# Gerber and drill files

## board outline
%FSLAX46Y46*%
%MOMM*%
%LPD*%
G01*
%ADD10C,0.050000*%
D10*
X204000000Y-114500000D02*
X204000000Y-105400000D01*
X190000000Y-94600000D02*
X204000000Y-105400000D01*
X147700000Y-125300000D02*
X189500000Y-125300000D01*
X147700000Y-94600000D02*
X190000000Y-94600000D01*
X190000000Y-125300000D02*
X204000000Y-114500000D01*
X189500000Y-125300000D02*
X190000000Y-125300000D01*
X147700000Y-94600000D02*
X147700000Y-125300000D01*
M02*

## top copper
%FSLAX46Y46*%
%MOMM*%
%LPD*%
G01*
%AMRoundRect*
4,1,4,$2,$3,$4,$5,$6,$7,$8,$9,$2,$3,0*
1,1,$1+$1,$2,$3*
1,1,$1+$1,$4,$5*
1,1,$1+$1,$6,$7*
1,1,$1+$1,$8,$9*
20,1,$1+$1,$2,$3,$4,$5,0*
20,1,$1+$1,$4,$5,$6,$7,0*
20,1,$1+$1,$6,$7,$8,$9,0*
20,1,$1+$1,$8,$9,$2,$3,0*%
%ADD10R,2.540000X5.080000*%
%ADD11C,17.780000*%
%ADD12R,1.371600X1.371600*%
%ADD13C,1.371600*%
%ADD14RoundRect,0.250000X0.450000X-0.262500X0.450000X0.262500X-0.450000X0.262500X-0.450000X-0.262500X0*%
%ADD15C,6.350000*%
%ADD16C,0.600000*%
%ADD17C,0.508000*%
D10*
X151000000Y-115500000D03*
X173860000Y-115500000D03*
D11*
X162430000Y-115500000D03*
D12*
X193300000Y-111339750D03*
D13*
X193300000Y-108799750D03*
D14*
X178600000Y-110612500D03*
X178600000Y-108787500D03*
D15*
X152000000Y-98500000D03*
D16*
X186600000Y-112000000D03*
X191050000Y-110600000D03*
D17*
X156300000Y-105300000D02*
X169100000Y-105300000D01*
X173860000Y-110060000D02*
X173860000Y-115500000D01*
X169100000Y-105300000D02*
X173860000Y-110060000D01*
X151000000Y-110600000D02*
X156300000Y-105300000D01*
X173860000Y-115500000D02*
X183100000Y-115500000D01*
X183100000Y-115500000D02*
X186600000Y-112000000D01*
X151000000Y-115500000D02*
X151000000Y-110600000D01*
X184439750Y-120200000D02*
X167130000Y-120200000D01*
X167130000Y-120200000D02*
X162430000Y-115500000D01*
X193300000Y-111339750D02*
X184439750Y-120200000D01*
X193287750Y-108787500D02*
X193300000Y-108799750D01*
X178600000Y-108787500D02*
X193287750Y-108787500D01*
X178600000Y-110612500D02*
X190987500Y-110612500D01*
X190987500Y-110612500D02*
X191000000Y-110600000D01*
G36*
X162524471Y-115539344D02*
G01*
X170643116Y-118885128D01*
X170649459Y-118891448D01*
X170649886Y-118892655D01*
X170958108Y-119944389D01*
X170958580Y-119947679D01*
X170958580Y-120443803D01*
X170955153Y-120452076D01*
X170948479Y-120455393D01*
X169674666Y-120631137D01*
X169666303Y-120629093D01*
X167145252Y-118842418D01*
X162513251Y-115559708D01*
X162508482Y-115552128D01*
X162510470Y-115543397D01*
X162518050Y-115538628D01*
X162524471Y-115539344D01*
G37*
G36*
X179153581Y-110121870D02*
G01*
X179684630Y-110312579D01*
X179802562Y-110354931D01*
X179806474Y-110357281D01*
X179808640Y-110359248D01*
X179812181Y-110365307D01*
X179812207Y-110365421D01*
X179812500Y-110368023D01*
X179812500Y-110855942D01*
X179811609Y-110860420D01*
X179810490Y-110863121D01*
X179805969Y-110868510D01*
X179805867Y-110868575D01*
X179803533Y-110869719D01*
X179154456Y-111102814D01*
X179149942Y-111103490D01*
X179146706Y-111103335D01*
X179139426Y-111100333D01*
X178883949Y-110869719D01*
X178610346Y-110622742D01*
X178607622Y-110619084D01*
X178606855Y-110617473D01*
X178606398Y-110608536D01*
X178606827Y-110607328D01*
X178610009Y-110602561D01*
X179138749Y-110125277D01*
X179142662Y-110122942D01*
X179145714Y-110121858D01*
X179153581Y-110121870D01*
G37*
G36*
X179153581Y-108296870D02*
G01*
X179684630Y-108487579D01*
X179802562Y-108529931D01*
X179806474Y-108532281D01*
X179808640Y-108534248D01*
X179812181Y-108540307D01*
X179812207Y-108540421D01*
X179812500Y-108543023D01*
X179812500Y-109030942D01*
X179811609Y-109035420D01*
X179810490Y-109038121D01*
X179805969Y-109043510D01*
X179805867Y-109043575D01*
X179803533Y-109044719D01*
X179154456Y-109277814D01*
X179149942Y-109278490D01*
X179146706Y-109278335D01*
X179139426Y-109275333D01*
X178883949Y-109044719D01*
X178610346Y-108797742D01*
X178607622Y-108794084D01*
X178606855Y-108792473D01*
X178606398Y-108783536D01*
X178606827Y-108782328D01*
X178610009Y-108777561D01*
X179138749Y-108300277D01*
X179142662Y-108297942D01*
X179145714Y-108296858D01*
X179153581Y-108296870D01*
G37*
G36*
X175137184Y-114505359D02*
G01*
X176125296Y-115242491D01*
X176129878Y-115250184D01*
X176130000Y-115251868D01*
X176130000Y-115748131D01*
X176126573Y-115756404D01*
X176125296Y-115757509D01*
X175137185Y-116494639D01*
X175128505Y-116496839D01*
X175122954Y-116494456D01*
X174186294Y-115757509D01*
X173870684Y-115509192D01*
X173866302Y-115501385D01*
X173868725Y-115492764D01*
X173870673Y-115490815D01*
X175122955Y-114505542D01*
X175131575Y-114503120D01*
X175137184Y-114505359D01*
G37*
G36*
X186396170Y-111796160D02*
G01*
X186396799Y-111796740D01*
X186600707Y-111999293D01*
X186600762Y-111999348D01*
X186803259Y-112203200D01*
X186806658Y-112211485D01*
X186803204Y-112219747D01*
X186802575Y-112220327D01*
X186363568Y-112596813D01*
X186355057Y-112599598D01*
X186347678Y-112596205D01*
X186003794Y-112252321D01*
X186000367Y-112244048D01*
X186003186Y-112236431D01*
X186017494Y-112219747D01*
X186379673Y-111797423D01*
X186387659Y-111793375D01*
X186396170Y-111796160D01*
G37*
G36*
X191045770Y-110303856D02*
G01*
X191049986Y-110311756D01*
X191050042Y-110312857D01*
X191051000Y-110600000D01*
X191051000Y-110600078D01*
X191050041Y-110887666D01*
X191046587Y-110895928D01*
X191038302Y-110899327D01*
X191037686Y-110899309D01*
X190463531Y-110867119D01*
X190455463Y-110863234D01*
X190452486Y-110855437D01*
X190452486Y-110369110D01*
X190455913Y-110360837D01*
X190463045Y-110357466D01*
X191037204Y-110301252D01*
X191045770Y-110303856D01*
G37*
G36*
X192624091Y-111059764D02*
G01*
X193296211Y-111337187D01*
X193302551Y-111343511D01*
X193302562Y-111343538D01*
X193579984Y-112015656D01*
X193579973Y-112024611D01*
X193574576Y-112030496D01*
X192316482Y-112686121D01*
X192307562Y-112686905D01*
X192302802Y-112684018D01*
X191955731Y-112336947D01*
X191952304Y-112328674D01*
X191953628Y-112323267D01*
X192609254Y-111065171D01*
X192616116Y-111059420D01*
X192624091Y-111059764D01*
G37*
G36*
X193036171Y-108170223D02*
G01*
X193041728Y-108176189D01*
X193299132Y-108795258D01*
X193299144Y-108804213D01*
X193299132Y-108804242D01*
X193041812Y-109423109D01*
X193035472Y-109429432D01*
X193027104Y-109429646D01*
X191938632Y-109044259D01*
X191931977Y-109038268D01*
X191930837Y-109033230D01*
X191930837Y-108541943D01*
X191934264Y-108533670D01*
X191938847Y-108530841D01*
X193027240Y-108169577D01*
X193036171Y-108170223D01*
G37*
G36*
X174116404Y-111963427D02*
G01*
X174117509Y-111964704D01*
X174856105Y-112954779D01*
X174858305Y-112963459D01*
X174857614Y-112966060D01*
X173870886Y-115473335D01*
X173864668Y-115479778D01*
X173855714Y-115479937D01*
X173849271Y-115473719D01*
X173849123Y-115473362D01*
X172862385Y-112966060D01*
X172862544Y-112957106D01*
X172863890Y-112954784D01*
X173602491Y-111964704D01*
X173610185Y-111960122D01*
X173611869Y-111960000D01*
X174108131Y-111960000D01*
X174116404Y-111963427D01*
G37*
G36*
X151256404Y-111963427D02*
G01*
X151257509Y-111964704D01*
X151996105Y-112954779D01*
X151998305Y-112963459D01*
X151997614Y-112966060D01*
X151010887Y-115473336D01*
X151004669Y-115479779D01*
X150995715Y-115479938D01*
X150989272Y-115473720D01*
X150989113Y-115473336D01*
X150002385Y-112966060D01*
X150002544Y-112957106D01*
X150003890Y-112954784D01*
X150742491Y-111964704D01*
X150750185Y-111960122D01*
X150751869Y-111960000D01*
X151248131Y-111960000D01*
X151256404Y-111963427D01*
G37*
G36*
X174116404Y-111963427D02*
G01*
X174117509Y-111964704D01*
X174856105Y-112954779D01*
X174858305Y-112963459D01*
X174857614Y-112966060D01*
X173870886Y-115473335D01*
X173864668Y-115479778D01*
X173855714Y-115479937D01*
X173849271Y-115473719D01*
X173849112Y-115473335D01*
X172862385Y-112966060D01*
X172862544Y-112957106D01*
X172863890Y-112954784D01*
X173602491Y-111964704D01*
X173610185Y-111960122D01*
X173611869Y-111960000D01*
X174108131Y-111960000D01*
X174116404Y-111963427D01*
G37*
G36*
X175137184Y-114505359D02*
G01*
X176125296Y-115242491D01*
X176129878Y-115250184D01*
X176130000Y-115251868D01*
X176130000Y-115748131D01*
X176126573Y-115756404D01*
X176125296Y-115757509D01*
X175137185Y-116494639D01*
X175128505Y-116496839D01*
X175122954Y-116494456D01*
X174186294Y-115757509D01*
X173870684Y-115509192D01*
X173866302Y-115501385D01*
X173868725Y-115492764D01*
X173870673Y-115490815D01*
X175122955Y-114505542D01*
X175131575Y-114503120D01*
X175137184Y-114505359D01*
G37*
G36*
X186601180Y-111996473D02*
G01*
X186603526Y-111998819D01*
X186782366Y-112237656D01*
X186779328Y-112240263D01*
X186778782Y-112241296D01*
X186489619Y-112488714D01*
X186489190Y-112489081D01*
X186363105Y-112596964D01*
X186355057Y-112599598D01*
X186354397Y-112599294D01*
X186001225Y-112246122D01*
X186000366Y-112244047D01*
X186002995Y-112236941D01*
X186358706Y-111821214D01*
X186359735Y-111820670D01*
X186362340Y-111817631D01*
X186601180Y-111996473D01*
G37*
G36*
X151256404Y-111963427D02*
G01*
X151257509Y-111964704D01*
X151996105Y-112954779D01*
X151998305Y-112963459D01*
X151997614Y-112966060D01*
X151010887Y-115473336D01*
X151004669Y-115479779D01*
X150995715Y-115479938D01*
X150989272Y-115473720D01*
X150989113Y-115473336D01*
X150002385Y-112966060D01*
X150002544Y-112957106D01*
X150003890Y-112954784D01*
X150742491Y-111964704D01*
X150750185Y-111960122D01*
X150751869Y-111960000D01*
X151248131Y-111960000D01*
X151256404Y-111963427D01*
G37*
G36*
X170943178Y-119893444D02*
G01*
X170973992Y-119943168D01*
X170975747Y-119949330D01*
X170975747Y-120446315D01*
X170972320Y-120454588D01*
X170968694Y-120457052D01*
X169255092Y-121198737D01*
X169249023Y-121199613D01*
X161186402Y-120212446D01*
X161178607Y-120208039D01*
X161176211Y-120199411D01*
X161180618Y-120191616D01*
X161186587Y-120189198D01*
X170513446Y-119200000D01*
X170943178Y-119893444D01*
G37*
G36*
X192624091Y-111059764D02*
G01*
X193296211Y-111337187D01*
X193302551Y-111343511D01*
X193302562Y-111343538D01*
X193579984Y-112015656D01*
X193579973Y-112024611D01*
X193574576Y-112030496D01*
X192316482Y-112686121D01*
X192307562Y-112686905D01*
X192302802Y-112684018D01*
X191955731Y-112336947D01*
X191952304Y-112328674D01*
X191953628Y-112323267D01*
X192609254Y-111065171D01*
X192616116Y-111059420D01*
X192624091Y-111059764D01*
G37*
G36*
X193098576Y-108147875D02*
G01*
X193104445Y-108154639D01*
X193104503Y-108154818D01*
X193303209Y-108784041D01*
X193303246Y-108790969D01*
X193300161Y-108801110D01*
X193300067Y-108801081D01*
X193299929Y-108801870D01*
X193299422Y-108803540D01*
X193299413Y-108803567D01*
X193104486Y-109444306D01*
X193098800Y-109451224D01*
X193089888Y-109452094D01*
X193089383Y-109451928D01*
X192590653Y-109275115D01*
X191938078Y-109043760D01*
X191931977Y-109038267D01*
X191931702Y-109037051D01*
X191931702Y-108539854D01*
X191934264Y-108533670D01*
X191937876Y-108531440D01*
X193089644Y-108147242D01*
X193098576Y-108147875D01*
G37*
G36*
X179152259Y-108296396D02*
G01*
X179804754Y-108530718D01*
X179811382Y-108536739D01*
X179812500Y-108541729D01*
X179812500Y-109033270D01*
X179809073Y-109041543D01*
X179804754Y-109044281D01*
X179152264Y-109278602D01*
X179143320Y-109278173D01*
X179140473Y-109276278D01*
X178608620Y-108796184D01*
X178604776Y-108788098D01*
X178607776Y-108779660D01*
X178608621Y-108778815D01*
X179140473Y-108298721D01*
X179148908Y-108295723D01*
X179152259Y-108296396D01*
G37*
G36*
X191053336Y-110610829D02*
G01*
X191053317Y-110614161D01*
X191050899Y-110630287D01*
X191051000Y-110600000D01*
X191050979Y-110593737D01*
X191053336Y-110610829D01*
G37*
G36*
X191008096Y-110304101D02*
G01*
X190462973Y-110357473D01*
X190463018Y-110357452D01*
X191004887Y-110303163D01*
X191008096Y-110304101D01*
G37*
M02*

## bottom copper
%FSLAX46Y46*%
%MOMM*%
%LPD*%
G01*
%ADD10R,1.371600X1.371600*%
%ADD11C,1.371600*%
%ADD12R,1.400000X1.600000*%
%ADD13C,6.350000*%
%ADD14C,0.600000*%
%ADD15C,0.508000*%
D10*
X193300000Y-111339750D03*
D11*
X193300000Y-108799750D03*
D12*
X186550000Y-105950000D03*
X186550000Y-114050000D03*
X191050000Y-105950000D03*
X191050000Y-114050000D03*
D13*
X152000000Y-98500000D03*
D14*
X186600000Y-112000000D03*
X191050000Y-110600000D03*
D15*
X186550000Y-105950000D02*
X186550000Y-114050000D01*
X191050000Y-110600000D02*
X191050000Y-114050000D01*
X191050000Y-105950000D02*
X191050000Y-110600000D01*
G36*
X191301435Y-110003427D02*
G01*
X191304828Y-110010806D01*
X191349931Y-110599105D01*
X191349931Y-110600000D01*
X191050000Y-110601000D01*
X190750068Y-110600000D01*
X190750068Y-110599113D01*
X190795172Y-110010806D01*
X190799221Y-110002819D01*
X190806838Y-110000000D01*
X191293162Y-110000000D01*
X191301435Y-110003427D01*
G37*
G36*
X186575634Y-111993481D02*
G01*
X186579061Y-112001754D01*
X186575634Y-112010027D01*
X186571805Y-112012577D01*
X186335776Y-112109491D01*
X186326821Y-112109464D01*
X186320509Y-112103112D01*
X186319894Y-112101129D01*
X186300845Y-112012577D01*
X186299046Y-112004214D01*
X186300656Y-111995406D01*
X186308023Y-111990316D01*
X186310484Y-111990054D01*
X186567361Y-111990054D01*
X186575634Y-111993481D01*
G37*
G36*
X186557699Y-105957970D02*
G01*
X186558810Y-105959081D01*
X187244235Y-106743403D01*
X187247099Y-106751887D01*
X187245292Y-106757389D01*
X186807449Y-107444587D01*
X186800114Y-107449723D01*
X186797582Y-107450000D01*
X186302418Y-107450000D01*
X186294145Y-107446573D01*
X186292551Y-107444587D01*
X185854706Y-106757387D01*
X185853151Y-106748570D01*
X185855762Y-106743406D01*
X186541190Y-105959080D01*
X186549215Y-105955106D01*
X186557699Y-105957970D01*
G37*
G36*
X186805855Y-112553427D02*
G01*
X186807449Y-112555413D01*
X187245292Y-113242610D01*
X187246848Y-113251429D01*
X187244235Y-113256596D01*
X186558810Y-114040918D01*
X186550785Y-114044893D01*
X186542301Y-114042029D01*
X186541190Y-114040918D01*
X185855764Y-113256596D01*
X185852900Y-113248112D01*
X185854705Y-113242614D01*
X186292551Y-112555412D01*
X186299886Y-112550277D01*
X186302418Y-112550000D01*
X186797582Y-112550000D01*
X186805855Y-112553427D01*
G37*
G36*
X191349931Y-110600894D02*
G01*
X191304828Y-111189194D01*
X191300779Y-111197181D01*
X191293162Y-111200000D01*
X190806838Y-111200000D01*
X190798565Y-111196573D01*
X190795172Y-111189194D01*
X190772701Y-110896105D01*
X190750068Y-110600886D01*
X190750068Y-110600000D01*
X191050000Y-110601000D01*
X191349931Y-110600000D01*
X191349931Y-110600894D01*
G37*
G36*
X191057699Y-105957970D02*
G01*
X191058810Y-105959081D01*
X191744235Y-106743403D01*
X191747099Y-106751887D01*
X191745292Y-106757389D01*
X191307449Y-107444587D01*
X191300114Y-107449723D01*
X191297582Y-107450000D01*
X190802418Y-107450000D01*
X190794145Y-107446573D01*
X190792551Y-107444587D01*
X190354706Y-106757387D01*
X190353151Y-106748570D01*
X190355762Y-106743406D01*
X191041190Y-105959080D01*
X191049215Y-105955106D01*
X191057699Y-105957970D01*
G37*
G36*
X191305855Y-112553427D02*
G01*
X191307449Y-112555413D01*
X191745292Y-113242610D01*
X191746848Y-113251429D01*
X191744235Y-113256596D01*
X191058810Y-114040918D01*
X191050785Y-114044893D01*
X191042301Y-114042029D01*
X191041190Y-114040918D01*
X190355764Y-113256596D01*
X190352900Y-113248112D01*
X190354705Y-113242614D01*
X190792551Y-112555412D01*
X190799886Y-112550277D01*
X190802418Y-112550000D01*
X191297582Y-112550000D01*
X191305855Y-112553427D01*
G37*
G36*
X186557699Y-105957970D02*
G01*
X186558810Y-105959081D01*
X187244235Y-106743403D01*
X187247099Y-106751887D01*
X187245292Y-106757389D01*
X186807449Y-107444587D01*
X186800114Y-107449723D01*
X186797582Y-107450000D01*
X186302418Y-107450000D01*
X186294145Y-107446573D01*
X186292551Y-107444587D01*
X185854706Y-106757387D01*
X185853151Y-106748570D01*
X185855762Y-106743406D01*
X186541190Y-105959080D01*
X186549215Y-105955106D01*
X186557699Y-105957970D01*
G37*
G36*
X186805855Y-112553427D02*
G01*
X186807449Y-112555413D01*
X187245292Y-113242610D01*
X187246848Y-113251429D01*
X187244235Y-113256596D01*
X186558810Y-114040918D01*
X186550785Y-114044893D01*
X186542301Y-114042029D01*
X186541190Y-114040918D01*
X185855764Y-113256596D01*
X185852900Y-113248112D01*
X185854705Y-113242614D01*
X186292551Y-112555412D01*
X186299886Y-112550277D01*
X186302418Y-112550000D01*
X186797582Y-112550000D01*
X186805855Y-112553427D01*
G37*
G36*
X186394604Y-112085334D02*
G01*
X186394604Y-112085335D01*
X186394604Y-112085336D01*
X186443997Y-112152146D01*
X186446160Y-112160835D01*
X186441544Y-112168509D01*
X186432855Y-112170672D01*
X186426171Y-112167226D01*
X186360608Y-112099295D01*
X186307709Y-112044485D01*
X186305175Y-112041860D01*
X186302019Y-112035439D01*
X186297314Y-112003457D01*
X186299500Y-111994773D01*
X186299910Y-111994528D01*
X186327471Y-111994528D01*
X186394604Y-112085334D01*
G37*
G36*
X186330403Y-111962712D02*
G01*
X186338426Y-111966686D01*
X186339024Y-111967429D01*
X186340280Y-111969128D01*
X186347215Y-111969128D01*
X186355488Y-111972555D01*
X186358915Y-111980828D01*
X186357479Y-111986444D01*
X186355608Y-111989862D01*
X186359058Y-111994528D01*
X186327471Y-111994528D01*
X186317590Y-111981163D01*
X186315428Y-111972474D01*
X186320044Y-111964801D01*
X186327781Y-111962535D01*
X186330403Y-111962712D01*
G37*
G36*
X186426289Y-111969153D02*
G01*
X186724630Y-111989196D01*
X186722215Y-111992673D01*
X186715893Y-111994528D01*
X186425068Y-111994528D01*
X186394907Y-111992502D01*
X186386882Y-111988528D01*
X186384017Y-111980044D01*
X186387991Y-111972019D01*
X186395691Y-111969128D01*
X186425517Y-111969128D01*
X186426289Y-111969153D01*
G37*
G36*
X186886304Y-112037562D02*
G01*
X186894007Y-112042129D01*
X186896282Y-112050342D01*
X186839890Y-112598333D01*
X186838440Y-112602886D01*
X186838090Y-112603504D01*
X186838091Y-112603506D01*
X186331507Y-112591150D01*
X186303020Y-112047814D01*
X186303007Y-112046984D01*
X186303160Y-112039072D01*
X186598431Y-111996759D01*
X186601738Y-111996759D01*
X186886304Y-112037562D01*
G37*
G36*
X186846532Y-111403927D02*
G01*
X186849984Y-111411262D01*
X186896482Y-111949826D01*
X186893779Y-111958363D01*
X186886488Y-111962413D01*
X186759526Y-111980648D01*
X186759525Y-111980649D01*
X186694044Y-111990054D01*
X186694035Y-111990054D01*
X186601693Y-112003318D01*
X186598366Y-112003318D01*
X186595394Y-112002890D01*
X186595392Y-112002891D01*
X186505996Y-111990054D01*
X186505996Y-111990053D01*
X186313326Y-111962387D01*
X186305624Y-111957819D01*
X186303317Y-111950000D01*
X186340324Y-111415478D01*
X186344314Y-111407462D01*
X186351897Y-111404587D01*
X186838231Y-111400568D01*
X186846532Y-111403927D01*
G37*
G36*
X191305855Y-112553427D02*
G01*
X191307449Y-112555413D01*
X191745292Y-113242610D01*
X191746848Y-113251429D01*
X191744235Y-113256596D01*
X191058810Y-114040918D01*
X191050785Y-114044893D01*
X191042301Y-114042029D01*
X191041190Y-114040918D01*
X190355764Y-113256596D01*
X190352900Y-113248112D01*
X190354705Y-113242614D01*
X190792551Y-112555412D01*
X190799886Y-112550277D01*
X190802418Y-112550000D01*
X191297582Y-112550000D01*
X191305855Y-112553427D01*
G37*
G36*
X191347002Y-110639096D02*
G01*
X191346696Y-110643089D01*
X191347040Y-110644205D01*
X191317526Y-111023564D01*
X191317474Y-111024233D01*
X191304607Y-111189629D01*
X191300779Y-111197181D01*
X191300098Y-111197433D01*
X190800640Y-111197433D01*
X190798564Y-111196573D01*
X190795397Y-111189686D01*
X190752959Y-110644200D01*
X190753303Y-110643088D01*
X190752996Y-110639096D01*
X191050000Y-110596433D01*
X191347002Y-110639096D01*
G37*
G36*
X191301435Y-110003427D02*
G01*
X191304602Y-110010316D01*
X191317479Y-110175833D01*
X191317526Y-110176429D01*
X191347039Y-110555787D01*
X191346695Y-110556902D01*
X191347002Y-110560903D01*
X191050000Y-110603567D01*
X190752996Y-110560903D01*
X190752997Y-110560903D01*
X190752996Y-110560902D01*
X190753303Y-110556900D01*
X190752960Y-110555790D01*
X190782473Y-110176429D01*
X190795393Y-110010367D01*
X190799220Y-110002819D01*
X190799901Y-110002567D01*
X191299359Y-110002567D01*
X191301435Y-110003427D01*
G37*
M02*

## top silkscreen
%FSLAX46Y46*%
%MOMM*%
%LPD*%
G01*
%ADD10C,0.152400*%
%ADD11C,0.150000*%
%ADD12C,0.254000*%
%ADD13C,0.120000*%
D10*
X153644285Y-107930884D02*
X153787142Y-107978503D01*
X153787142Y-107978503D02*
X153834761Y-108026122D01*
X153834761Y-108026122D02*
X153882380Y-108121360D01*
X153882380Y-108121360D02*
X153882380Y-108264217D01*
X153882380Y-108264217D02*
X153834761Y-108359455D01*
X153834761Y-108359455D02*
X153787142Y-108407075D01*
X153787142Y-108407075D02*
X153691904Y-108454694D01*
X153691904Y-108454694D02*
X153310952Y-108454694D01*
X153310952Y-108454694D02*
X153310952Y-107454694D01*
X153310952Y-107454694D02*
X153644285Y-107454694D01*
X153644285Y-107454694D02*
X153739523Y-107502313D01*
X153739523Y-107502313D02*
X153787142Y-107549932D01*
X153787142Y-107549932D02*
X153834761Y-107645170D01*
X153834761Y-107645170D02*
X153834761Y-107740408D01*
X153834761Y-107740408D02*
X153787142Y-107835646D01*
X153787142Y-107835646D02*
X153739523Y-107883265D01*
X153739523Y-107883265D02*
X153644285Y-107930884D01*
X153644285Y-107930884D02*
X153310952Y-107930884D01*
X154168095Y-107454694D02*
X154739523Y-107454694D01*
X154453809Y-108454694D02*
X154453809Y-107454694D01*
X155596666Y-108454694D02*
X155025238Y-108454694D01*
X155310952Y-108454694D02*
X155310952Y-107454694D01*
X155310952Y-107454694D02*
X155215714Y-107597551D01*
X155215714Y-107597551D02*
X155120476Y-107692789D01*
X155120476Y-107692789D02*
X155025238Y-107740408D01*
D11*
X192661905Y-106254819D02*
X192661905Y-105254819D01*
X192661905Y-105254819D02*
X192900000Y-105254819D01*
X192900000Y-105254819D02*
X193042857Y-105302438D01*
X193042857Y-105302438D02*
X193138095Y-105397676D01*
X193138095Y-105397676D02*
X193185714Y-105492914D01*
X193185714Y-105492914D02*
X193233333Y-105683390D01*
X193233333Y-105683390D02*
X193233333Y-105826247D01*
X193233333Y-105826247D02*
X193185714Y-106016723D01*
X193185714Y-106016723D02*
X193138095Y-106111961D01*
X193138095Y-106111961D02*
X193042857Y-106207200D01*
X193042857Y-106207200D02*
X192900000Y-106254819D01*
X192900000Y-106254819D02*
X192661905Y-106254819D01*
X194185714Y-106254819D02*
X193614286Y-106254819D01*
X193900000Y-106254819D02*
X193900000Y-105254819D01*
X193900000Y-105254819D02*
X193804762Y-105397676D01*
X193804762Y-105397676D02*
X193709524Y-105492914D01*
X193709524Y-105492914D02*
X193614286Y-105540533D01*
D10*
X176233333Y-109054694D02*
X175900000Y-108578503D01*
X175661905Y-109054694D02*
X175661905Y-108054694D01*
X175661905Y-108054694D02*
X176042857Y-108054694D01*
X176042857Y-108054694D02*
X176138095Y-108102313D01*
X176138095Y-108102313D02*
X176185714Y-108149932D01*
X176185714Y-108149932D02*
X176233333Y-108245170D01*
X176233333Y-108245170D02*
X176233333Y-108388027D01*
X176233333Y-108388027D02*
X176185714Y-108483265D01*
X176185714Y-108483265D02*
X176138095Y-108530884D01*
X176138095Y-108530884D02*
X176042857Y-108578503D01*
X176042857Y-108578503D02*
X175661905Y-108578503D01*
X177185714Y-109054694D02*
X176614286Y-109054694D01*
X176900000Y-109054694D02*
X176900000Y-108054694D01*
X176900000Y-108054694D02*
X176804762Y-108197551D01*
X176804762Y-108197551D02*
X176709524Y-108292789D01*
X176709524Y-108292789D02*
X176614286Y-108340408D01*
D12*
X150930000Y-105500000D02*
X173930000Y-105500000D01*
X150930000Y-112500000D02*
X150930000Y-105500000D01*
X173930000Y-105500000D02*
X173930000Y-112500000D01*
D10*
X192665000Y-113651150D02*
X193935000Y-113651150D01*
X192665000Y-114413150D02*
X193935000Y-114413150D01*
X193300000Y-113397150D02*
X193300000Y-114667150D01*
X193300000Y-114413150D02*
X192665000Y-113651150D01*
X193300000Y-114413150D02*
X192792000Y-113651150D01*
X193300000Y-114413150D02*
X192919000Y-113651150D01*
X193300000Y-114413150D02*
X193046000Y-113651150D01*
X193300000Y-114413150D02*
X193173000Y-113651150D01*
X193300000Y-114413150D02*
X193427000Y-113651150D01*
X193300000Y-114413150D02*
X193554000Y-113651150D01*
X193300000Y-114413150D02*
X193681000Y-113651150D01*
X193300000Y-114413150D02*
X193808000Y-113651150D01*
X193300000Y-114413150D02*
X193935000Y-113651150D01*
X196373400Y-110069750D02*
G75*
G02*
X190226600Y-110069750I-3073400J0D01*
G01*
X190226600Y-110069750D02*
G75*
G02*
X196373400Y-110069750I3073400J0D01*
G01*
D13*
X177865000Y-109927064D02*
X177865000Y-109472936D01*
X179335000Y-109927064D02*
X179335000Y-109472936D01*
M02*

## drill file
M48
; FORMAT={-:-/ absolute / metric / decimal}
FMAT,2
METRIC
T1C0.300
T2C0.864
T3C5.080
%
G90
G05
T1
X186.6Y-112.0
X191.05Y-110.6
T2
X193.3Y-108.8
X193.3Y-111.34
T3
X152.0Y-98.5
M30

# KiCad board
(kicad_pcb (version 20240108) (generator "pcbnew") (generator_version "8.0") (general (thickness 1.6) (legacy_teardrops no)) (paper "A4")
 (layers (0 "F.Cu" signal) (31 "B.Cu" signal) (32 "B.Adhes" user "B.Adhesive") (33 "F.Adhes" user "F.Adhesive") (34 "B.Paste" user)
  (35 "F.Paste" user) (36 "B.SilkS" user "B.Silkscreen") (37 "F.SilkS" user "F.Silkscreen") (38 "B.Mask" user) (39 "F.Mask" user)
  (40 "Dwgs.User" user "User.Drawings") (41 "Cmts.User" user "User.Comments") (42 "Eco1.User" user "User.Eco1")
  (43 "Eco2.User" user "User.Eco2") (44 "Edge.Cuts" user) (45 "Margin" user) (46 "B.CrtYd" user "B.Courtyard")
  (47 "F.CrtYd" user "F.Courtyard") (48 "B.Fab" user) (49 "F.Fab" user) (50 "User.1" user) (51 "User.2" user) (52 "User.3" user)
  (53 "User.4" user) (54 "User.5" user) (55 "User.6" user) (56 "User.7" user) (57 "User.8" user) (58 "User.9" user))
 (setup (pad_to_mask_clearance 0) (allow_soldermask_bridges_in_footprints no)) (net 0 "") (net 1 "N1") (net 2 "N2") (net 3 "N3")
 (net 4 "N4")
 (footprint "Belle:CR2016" (layer "F.Cu") (at 162.43 115.5)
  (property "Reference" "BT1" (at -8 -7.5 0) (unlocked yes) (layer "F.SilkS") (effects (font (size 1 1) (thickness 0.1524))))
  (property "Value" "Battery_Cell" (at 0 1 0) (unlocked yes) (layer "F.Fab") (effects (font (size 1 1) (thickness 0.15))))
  (fp_line (start -11.5 -10) (end 11.5 -10) (stroke (width 0.254) (type default)) (layer "F.SilkS"))
  (fp_line (start -11.5 -3) (end -11.5 -10) (stroke (width 0.254) (type default)) (layer "F.SilkS"))
  (fp_line (start 11.5 -10) (end 11.5 -3) (stroke (width 0.254) (type default)) (layer "F.SilkS"))
  (pad "1" smd rect (at -11.43 0) (size 2.54 5.08) (layers "F.Cu" "F.Paste" "F.Mask") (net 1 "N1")
   (teardrops (best_length_ratio 0.5) (max_length 1) (best_width_ratio 1) (max_width 2) (curve_points 0) (filter_ratio 0.9) (enabled yes)
    (allow_two_segments yes) (prefer_zone_connections yes)))
  (pad "1" smd rect (at 11.43 0) (size 2.54 5.08) (layers "F.Cu" "F.Paste" "F.Mask") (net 1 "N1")
   (teardrops (best_length_ratio 0.5) (max_length 1) (best_width_ratio 1) (max_width 2) (curve_points 0) (filter_ratio 0.9) (enabled yes)
    (allow_two_segments yes) (prefer_zone_connections yes)))
  (pad "2" smd circle (at 0 0) (size 17.78 17.78) (layers "F.Cu" "F.Paste" "F.Mask") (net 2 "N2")
   (teardrops (best_length_ratio 0.5) (max_length 1) (best_width_ratio 1) (max_width 2) (curve_points 0) (filter_ratio 0.9) (enabled yes)
    (allow_two_segments yes) (prefer_zone_connections yes))))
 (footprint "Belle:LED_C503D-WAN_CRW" (layer "F.Cu") (at 193.3 111.33975 90)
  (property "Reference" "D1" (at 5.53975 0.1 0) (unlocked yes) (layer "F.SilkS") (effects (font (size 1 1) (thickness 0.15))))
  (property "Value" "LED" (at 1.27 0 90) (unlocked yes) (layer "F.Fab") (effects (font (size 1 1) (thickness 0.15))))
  (fp_line (start -2.3114 -0.635) (end -2.3114 0.635) (stroke (width 0.1524) (type solid)) (layer "F.SilkS"))
  (fp_line (start -3.0734 -0.635) (end -3.0734 0.635) (stroke (width 0.1524) (type solid)) (layer "F.SilkS"))
  (fp_line (start -2.0574 0) (end -3.3274 0) (stroke (width 0.1524) (type solid)) (layer "F.SilkS"))
  (fp_line (start -3.0734 0) (end -2.3114 -0.635) (stroke (width 0.1524) (type solid)) (layer "F.SilkS"))
  (fp_line (start -3.0734 0) (end -2.3114 -0.508) (stroke (width 0.1524) (type solid)) (layer "F.SilkS"))
  (fp_line (start -3.0734 0) (end -2.3114 -0.381) (stroke (width 0.1524) (type solid)) (layer "F.SilkS"))
  (fp_line (start -3.0734 0) (end -2.3114 -0.254) (stroke (width 0.1524) (type solid)) (layer "F.SilkS"))
  (fp_line (start -3.0734 0) (end -2.3114 -0.127) (stroke (width 0.1524) (type solid)) (layer "F.SilkS"))
  (fp_line (start -3.0734 0) (end -2.3114 0.127) (stroke (width 0.1524) (type solid)) (layer "F.SilkS"))
  (fp_line (start -3.0734 0) (end -2.3114 0.254) (stroke (width 0.1524) (type solid)) (layer "F.SilkS"))
  (fp_line (start -3.0734 0) (end -2.3114 0.381) (stroke (width 0.1524) (type solid)) (layer "F.SilkS"))
  (fp_line (start -3.0734 0) (end -2.3114 0.508) (stroke (width 0.1524) (type solid)) (layer "F.SilkS"))
  (fp_line (start -3.0734 0) (end -2.3114 0.635) (stroke (width 0.1524) (type solid)) (layer "F.SilkS"))
  (fp_circle (center 1.27 0) (end 4.3434 0) (stroke (width 0.1524) (type solid)) (fill none) (layer "F.SilkS"))
  (pad "1" thru_hole rect (at 0 0 90) (size 1.3716 1.3716) (drill 0.8636) (layers "*.Cu" "*.Mask") (remove_unused_layers no) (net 2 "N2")
   (teardrops (best_length_ratio 0.5) (max_length 1) (best_width_ratio 1) (max_width 2) (curve_points 0) (filter_ratio 0.9) (enabled yes)
    (allow_two_segments yes) (prefer_zone_connections yes)))
  (pad "2" thru_hole circle (at 2.54 0 90) (size 1.3716 1.3716) (drill 0.8636) (layers "*.Cu" "*.Mask") (remove_unused_layers no)
   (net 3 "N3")
   (teardrops (best_length_ratio 0.5) (max_length 1) (best_width_ratio 1) (max_width 2) (curve_points 0) (filter_ratio 0.9) (enabled yes)
    (allow_two_segments yes) (prefer_zone_connections yes))))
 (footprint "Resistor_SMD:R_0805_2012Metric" (layer "F.Cu") (at 178.6 109.7 90)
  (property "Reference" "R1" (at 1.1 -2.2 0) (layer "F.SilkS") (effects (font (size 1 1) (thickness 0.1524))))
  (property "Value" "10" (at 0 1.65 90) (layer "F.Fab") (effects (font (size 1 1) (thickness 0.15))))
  (fp_line (start -0.227064 -0.735) (end 0.227064 -0.735) (stroke (width 0.12) (type solid)) (layer "F.SilkS"))
  (fp_line (start -0.227064 0.735) (end 0.227064 0.735) (stroke (width 0.12) (type solid)) (layer "F.SilkS"))
  (pad "1" smd roundrect (at -0.9125 0 90) (size 1.025 1.4) (layers "F.Cu" "F.Paste" "F.Mask") (roundrect_rratio 0.243902) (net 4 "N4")
   (teardrops (best_length_ratio 0.5) (max_length 1) (best_width_ratio 1) (max_width 2) (curve_points 0) (filter_ratio 0.9) (enabled yes)
    (allow_two_segments yes) (prefer_zone_connections yes)))
  (pad "2" smd roundrect (at 0.9125 0 90) (size 1.025 1.4) (layers "F.Cu" "F.Paste" "F.Mask") (roundrect_rratio 0.243902) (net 3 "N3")
   (teardrops (best_length_ratio 0.5) (max_length 1) (best_width_ratio 1) (max_width 2) (curve_points 0) (filter_ratio 0.9) (enabled yes)
    (allow_two_segments yes) (prefer_zone_connections yes))))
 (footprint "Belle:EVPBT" (layer "B.Cu") (at 188.8 110 -90)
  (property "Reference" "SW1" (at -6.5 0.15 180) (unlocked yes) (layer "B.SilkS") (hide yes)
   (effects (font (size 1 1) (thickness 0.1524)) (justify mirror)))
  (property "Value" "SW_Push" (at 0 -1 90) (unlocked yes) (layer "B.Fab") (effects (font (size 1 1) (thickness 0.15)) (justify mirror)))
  (pad "1" smd rect (at -4.05 2.25 270) (size 1.6 1.4) (layers "B.Cu" "B.Paste" "B.Mask") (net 1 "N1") (thermal_bridge_angle 45)
   (teardrops (best_length_ratio 0.5) (max_length 1) (best_width_ratio 1) (max_width 2) (curve_points 0) (filter_ratio 0.9) (enabled yes)
    (allow_two_segments yes) (prefer_zone_connections yes)))
  (pad "1" smd rect (at 4.05 2.25 270) (size 1.6 1.4) (layers "B.Cu" "B.Paste" "B.Mask") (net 1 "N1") (thermal_bridge_angle 45)
   (teardrops (best_length_ratio 0.5) (max_length 1) (best_width_ratio 1) (max_width 2) (curve_points 0) (filter_ratio 0.9) (enabled yes)
    (allow_two_segments yes) (prefer_zone_connections yes)))
  (pad "2" smd rect (at -4.05 -2.25 270) (size 1.6 1.4) (layers "B.Cu" "B.Paste" "B.Mask") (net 4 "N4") (thermal_bridge_angle 45)
   (teardrops (best_length_ratio 0.5) (max_length 1) (best_width_ratio 1) (max_width 2) (curve_points 0) (filter_ratio 0.9) (enabled yes)
    (allow_two_segments yes) (prefer_zone_connections yes)))
  (pad "2" smd rect (at 4.05 -2.25 270) (size 1.6 1.4) (layers "B.Cu" "B.Paste" "B.Mask") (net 4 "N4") (thermal_bridge_angle 45)
   (teardrops (best_length_ratio 0.5) (max_length 1) (best_width_ratio 1) (max_width 2) (curve_points 0) (filter_ratio 0.9) (enabled yes)
    (allow_two_segments yes) (prefer_zone_connections yes))))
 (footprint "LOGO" (layer "B.Cu") (at 166.448159 109.511349 180)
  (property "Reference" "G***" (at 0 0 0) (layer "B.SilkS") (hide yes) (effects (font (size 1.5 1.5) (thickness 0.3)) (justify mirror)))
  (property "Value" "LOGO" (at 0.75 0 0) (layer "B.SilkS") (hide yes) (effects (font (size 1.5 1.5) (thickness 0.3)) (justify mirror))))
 (gr_line (start 204 114.5) (end 204 105.4) (stroke (width 0.05) (type default)) (layer "Edge.Cuts"))
 (gr_line (start 190 94.6) (end 204 105.4) (stroke (width 0.05) (type default)) (layer "Edge.Cuts"))
 (gr_line (start 147.7 125.3) (end 189.5 125.3) (stroke (width 0.05) (type default)) (layer "Edge.Cuts"))
 (gr_line (start 147.7 94.6) (end 190 94.6) (stroke (width 0.05) (type default)) (layer "Edge.Cuts"))
 (gr_line (start 190 125.3) (end 204 114.5) (stroke (width 0.05) (type default)) (layer "Edge.Cuts"))
 (gr_line (start 189.5 125.3) (end 190 125.3) (stroke (width 0.05) (type default)) (layer "Edge.Cuts"))
 (gr_line (start 147.7 94.6) (end 147.7 125.3) (stroke (width 0.05) (type default)) (layer "Edge.Cuts"))
 (via (at 152 98.5) (size 6.35) (drill 5.08) (layers "F.Cu" "B.Cu")
  (teardrops (best_length_ratio 0.5) (max_length 1) (best_width_ratio 1) (max_width 2) (curve_points 0) (filter_ratio 0.9) (enabled yes)
   (allow_two_segments yes) (prefer_zone_connections yes))
  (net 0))
 (segment (start 156.3 105.3) (end 169.1 105.3) (width 0.508) (layer "F.Cu") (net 1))
 (segment (start 173.86 110.06) (end 173.86 115.5) (width 0.508) (layer "F.Cu") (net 1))
 (segment (start 169.1 105.3) (end 173.86 110.06) (width 0.508) (layer "F.Cu") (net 1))
 (segment (start 151 110.6) (end 156.3 105.3) (width 0.508) (layer "F.Cu") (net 1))
 (segment (start 173.86 115.5) (end 183.1 115.5) (width 0.508) (layer "F.Cu") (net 1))
 (segment (start 183.1 115.5) (end 186.6 112) (width 0.508) (layer "F.Cu") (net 1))
 (segment (start 151 115.5) (end 151 110.6) (width 0.508) (layer "F.Cu") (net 1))
 (via (at 186.6 112) (size 0.6) (drill 0.3) (layers "F.Cu" "B.Cu")
  (teardrops (best_length_ratio 0.5) (max_length 1) (best_width_ratio 1) (max_width 2) (curve_points 0) (filter_ratio 0.9) (enabled yes)
   (allow_two_segments yes) (prefer_zone_connections yes))
  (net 1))
 (segment (start 186.55 105.95) (end 186.55 114.05) (width 0.508) (layer "B.Cu") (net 1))
 (segment (start 184.43975 120.2) (end 167.13 120.2) (width 0.508) (layer "F.Cu") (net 2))
 (segment (start 167.13 120.2) (end 162.43 115.5) (width 0.508) (layer "F.Cu") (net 2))
 (segment (start 193.3 111.33975) (end 184.43975 120.2) (width 0.508) (layer "F.Cu") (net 2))
 (segment (start 193.28775 108.7875) (end 193.3 108.79975) (width 0.508) (layer "F.Cu") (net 3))
 (segment (start 178.6 108.7875) (end 193.28775 108.7875) (width 0.508) (layer "F.Cu") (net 3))
 (segment (start 178.6 110.6125) (end 190.9875 110.6125) (width 0.508) (layer "F.Cu") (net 4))
 (segment (start 190.9875 110.6125) (end 191 110.6) (width 0.508) (layer "F.Cu") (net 4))
 (via (at 191.05 110.6) (size 0.6) (drill 0.3) (layers "F.Cu" "B.Cu")
  (teardrops (best_length_ratio 0.5) (max_length 1) (best_width_ratio 1) (max_width 2) (curve_points 0) (filter_ratio 0.9) (enabled yes)
   (allow_two_segments yes) (prefer_zone_connections yes))
  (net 4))
 (segment (start 191.05 110.6) (end 191.05 114.05) (width 0.508) (layer "B.Cu") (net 4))
 (segment (start 191.05 105.95) (end 191.05 110.6) (width 0.508) (layer "B.Cu") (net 4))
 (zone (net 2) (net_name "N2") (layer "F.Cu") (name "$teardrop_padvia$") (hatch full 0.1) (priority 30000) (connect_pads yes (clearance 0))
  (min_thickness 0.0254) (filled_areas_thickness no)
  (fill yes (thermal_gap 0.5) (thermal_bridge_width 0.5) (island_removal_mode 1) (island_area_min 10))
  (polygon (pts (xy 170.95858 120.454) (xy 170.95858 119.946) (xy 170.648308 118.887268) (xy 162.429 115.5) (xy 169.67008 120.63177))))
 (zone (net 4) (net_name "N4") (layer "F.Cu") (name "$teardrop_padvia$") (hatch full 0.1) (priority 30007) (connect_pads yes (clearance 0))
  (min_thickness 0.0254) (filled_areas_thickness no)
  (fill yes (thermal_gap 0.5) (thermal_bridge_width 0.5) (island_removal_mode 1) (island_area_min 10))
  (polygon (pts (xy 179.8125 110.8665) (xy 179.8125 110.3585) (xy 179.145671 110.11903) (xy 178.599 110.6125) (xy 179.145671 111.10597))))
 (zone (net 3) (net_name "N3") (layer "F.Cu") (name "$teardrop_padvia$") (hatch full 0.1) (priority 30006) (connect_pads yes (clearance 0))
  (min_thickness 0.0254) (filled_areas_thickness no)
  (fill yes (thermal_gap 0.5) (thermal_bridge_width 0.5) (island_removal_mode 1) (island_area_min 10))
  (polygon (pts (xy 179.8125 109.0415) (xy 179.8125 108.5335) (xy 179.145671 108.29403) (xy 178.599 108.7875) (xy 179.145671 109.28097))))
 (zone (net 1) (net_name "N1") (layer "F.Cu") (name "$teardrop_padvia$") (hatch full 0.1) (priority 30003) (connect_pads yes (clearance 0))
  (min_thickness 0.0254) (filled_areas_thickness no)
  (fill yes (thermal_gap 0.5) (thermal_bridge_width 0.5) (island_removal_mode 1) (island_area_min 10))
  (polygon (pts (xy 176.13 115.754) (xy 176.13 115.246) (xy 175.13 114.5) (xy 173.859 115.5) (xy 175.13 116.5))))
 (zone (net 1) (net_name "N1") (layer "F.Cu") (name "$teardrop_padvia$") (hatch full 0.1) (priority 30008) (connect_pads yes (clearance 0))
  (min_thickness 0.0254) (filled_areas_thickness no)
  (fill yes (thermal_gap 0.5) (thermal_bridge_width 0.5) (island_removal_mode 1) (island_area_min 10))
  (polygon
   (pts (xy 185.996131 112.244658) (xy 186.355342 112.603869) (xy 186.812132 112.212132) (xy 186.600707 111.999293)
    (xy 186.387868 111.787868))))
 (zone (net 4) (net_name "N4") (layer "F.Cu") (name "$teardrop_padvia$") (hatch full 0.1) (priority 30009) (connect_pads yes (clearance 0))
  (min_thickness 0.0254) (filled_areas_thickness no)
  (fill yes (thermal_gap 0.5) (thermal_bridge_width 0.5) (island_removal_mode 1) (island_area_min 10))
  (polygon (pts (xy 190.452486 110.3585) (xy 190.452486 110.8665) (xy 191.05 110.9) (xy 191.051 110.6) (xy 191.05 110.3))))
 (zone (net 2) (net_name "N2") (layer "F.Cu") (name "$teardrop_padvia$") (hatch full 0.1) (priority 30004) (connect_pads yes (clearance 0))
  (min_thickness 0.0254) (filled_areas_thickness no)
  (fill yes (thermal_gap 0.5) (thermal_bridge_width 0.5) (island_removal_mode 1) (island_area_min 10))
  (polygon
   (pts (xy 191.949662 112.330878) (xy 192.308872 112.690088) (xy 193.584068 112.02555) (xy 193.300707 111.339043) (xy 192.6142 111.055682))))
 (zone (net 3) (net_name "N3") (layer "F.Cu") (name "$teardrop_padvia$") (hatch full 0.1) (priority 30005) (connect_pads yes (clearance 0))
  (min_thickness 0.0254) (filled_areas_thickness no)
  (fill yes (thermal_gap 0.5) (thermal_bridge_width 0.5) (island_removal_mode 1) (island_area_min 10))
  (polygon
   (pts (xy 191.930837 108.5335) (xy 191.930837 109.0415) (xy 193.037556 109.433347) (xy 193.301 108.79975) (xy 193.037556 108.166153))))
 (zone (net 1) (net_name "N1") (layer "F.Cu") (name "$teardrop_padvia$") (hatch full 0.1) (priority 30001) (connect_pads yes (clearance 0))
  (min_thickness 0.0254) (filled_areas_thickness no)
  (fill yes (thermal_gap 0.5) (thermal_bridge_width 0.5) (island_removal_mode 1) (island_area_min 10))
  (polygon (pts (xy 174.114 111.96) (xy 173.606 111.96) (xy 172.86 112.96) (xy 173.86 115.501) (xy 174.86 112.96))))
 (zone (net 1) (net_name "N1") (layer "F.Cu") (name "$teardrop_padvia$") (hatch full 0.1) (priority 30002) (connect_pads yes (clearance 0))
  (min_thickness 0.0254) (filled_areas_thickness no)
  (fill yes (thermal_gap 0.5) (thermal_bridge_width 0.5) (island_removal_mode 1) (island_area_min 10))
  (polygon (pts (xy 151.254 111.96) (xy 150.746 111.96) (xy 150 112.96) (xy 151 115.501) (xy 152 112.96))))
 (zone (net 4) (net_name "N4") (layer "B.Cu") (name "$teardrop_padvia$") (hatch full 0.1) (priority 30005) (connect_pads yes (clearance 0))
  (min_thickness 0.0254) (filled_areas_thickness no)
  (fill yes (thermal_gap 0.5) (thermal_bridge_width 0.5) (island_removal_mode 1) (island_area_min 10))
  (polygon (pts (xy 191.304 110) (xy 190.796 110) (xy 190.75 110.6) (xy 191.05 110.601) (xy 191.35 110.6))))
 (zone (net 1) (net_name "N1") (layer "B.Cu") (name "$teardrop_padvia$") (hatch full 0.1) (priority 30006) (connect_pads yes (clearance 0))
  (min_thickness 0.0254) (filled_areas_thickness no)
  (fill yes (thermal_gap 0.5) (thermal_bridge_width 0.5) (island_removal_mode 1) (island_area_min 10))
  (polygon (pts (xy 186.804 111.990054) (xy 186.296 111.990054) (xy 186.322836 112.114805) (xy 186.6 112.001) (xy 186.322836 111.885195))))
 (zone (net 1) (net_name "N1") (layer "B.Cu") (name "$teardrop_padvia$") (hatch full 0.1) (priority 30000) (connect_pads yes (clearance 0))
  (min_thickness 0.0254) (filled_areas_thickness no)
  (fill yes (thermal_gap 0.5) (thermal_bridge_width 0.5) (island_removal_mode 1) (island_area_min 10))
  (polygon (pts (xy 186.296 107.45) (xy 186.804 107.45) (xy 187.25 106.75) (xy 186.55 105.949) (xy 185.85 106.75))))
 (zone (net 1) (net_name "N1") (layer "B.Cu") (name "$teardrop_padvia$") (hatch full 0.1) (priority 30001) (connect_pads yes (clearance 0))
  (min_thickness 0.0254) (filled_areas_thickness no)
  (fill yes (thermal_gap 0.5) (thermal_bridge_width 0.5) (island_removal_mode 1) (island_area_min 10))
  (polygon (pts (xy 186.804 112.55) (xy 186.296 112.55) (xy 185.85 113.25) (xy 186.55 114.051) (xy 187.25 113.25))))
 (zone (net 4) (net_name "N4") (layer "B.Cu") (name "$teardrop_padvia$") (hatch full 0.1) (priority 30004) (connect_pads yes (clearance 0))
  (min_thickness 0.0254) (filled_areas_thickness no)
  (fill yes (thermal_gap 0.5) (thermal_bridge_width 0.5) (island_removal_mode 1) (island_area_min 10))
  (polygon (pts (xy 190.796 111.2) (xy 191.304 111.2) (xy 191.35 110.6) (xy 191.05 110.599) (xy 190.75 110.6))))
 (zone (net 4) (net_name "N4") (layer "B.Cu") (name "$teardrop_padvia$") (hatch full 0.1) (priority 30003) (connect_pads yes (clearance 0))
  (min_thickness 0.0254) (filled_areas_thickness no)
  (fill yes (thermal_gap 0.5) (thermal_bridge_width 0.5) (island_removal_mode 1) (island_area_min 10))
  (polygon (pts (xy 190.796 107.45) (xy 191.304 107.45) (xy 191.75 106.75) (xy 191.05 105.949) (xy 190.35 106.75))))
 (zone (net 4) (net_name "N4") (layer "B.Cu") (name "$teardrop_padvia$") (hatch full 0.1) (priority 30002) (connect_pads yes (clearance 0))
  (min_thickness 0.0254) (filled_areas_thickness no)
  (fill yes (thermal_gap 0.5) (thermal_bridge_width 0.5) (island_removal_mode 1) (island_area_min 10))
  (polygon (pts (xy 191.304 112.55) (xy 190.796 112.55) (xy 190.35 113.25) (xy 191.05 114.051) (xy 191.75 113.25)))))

